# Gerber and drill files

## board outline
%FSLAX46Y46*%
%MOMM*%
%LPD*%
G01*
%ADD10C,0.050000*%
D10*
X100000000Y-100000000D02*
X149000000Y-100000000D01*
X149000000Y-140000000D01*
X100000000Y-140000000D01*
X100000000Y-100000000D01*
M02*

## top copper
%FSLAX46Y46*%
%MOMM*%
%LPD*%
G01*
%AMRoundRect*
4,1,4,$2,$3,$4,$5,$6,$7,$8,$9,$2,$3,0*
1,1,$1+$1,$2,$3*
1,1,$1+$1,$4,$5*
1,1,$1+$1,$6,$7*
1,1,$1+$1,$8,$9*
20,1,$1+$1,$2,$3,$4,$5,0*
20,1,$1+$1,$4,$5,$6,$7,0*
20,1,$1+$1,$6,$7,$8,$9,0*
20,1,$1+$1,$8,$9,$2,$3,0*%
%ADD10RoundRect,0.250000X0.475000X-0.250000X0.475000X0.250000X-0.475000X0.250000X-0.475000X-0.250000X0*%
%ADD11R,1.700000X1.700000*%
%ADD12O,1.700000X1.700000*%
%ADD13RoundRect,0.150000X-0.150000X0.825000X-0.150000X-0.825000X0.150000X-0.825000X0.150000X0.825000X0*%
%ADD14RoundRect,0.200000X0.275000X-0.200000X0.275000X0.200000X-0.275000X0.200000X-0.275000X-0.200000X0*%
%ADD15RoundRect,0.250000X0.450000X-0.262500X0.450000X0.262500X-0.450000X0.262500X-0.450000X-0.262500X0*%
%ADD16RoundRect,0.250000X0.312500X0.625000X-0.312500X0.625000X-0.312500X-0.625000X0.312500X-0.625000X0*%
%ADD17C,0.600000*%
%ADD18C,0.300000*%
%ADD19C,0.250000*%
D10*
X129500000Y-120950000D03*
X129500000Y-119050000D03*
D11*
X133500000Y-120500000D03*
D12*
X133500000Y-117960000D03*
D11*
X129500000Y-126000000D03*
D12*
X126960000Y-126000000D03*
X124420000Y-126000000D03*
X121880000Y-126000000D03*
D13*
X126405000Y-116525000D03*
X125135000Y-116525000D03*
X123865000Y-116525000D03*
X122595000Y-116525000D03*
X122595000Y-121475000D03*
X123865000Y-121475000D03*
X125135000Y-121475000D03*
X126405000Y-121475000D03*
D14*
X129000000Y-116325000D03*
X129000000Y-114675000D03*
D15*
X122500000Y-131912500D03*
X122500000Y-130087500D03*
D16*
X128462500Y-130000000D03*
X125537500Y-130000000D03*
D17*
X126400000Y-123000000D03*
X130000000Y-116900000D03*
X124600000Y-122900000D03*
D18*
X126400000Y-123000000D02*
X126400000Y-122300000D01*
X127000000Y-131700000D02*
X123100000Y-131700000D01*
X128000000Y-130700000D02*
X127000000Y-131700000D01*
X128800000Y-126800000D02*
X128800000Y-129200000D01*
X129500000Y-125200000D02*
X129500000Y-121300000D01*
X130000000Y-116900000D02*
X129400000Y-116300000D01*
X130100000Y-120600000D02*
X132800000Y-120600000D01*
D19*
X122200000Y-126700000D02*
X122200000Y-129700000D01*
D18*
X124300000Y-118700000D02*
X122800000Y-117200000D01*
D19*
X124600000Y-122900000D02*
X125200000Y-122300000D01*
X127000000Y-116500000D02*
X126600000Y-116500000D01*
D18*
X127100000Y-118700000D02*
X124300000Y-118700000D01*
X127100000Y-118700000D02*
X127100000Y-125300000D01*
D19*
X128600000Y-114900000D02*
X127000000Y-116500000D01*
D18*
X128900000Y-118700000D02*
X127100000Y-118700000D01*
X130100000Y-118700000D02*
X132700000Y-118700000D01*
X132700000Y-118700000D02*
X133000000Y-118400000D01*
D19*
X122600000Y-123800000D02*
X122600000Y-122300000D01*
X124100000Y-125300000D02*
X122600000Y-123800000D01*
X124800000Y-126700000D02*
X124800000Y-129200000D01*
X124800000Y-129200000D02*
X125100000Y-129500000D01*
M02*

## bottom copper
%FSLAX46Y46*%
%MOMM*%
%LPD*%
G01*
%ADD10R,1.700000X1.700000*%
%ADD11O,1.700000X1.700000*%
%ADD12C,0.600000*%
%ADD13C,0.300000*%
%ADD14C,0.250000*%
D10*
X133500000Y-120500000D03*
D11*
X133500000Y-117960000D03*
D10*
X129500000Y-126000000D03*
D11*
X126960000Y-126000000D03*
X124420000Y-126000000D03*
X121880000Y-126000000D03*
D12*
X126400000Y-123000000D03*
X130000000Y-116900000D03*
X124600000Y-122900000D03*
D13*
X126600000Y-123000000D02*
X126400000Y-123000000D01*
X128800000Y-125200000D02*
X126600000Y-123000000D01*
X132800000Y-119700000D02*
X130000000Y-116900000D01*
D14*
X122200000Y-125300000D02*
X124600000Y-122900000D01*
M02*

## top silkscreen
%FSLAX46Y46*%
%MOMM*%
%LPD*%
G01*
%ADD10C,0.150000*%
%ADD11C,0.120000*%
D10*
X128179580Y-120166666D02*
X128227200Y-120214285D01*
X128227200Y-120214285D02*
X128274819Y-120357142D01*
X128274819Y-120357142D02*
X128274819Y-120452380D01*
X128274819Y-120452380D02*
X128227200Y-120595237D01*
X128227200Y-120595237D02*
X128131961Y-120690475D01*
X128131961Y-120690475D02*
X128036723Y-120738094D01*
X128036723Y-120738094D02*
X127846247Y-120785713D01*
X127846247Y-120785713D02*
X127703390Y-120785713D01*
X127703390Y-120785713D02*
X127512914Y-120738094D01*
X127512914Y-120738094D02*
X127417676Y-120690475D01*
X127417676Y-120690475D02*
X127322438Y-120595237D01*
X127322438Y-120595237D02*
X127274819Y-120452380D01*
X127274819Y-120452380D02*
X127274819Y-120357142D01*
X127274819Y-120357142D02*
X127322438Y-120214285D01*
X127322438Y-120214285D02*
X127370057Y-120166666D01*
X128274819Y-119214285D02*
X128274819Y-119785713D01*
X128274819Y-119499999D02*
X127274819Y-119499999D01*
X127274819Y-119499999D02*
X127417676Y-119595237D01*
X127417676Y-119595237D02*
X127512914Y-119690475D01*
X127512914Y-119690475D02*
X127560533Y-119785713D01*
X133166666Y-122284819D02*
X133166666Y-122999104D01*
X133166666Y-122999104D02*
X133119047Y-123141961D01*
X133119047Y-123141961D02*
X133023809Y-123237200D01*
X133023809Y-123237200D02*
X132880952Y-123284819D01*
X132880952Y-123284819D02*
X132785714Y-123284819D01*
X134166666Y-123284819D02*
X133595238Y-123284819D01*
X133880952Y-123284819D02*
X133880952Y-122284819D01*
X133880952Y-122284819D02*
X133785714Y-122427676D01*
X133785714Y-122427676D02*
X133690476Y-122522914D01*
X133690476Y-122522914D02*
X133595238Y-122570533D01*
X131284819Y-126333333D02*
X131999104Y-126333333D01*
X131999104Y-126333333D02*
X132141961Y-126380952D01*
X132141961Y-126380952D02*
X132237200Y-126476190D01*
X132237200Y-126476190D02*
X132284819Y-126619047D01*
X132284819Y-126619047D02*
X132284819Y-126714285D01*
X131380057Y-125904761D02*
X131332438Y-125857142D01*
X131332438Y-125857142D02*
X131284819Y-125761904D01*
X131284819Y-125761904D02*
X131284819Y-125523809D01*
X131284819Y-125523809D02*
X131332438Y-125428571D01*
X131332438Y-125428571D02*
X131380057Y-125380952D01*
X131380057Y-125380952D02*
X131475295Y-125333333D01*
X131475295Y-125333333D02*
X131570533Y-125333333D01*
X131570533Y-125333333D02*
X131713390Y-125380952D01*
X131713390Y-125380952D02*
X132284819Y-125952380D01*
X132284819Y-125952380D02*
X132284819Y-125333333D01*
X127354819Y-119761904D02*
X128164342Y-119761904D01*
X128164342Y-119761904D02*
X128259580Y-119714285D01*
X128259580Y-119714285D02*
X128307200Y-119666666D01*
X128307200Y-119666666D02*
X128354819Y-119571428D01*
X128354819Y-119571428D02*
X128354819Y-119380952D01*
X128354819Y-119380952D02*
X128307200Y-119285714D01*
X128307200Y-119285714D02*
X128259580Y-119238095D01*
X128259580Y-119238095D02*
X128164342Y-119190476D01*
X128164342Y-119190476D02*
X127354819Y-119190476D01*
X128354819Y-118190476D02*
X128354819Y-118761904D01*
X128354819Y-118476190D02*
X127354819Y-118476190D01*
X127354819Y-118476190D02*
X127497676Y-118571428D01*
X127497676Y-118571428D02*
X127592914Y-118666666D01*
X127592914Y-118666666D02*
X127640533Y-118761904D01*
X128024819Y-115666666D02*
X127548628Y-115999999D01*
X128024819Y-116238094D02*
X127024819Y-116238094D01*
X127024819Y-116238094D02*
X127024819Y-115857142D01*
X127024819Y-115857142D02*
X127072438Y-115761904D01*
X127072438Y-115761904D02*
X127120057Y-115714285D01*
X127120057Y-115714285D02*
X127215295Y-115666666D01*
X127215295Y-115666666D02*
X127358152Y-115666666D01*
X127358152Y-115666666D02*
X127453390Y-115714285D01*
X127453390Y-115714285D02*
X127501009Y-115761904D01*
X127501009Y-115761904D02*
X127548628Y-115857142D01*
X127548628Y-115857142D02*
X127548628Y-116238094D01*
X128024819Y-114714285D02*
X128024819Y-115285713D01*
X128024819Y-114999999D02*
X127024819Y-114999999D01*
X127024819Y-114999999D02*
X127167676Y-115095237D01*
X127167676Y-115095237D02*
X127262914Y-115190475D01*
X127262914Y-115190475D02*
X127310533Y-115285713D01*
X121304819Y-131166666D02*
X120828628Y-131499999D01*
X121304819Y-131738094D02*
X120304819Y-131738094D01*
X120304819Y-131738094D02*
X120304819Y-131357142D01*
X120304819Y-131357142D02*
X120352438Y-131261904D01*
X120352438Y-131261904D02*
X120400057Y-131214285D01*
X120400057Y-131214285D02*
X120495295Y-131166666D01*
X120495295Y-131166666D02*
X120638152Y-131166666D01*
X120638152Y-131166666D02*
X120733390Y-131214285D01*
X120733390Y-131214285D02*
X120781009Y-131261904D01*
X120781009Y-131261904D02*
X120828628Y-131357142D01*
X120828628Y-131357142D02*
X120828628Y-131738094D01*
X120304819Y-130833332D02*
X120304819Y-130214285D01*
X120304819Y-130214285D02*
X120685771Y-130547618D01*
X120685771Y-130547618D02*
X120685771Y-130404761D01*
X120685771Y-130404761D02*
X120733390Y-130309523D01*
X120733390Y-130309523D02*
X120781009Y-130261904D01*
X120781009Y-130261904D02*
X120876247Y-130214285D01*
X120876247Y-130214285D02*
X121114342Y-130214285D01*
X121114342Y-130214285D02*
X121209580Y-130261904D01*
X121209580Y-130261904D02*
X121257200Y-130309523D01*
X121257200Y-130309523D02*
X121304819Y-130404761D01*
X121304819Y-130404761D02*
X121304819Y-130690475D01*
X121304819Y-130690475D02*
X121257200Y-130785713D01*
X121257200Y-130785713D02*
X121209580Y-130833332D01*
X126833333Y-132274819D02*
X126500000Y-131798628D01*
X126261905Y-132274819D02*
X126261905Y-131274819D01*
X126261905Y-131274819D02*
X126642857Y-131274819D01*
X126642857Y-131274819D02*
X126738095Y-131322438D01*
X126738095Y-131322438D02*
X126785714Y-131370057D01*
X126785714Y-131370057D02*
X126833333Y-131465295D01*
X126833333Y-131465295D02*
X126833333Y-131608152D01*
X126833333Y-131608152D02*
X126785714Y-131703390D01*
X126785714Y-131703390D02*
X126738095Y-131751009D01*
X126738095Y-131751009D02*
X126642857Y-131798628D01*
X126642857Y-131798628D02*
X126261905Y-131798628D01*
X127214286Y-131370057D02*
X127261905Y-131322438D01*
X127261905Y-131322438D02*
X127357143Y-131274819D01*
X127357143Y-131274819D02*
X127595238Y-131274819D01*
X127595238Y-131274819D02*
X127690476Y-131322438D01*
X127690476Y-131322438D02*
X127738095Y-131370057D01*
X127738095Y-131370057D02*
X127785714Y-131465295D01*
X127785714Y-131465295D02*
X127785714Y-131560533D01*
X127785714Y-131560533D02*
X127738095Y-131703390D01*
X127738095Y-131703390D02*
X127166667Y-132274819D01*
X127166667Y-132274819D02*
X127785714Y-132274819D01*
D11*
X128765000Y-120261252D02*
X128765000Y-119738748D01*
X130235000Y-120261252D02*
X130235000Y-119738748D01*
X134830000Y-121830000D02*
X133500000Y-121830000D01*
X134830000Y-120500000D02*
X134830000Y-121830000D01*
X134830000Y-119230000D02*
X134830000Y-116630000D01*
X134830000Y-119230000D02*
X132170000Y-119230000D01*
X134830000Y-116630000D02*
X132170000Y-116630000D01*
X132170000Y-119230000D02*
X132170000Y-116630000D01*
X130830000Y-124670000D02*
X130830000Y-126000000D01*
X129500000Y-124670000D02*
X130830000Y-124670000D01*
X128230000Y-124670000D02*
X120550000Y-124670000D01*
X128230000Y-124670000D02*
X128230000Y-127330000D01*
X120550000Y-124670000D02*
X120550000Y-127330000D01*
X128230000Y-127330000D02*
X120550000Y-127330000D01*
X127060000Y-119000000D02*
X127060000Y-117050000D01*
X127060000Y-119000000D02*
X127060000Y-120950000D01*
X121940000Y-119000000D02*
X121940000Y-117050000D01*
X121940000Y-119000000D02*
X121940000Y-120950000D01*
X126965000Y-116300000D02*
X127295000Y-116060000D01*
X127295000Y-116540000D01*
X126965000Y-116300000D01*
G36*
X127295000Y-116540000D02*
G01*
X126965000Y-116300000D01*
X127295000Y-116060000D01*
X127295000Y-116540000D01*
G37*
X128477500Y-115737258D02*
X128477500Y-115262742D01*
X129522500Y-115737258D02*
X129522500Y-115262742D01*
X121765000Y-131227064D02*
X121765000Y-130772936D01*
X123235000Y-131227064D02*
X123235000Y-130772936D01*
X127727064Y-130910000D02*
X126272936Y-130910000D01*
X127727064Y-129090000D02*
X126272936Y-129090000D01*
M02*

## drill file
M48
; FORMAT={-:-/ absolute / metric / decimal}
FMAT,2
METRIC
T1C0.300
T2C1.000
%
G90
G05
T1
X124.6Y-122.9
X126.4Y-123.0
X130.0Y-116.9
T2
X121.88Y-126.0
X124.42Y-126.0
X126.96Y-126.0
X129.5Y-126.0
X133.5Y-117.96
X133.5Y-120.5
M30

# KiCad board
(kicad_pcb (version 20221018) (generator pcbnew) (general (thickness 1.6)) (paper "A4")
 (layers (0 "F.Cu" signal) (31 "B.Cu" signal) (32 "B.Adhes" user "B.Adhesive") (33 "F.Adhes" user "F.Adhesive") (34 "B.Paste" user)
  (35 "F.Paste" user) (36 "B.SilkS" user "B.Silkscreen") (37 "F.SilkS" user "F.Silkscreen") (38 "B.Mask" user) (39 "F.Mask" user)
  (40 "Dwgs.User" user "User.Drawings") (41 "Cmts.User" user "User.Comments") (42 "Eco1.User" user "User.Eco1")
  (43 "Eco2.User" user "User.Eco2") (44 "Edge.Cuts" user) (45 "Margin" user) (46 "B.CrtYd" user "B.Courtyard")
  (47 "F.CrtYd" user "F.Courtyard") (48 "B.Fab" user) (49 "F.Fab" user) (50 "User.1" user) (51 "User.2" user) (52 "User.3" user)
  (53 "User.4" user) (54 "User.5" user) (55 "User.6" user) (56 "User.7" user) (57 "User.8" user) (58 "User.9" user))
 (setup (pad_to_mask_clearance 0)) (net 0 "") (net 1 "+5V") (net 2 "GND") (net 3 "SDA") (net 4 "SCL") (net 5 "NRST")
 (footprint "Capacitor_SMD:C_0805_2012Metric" (layer "F.Cu") (at 129.5 120 90)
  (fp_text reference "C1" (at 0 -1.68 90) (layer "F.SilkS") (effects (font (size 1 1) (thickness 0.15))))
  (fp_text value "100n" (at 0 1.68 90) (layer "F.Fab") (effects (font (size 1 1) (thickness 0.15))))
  (fp_line (start -0.261252 -0.735) (end 0.261252 -0.735) (stroke (width 0.12) (type solid)) (layer "F.SilkS"))
  (fp_line (start -0.261252 0.735) (end 0.261252 0.735) (stroke (width 0.12) (type solid)) (layer "F.SilkS"))
  (pad "1" smd roundrect (at -0.95 0 90) (size 1 1.45) (layers "F.Cu" "F.Paste" "F.Mask") (roundrect_rratio 0.25) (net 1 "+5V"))
  (pad "2" smd roundrect (at 0.95 0 90) (size 1 1.45) (layers "F.Cu" "F.Paste" "F.Mask") (roundrect_rratio 0.25) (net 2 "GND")))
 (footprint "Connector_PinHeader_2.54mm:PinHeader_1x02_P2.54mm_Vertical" (layer "F.Cu") (at 133.5 120.5 180)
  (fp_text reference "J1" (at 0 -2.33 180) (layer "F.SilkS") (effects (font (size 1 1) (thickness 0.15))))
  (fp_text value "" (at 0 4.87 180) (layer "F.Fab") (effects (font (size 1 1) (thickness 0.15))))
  (fp_line (start -1.33 -1.33) (end 0 -1.33) (stroke (width 0.12) (type solid)) (layer "F.SilkS"))
  (fp_line (start -1.33 0) (end -1.33 -1.33) (stroke (width 0.12) (type solid)) (layer "F.SilkS"))
  (fp_line (start -1.33 1.27) (end -1.33 3.87) (stroke (width 0.12) (type solid)) (layer "F.SilkS"))
  (fp_line (start -1.33 1.27) (end 1.33 1.27) (stroke (width 0.12) (type solid)) (layer "F.SilkS"))
  (fp_line (start -1.33 3.87) (end 1.33 3.87) (stroke (width 0.12) (type solid)) (layer "F.SilkS"))
  (fp_line (start 1.33 1.27) (end 1.33 3.87) (stroke (width 0.12) (type solid)) (layer "F.SilkS"))
  (pad "1" thru_hole rect (at 0 0 180) (size 1.7 1.7) (drill 1) (layers "*.Cu" "*.Mask") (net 1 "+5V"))
  (pad "2" thru_hole oval (at 0 2.54 180) (size 1.7 1.7) (drill 1) (layers "*.Cu" "*.Mask") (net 2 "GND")))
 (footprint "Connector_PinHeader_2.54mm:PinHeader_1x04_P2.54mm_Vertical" (layer "F.Cu") (at 129.5 126 -90)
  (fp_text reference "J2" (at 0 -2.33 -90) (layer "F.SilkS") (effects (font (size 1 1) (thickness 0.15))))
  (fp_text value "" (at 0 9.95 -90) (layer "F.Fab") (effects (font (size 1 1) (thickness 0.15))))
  (fp_line (start -1.33 -1.33) (end 0 -1.33) (stroke (width 0.12) (type solid)) (layer "F.SilkS"))
  (fp_line (start -1.33 0) (end -1.33 -1.33) (stroke (width 0.12) (type solid)) (layer "F.SilkS"))
  (fp_line (start -1.33 1.27) (end -1.33 8.95) (stroke (width 0.12) (type solid)) (layer "F.SilkS"))
  (fp_line (start -1.33 1.27) (end 1.33 1.27) (stroke (width 0.12) (type solid)) (layer "F.SilkS"))
  (fp_line (start -1.33 8.95) (end 1.33 8.95) (stroke (width 0.12) (type solid)) (layer "F.SilkS"))
  (fp_line (start 1.33 1.27) (end 1.33 8.95) (stroke (width 0.12) (type solid)) (layer "F.SilkS"))
  (pad "1" thru_hole rect (at 0 0 270) (size 1.7 1.7) (drill 1) (layers "*.Cu" "*.Mask") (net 1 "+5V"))
  (pad "2" thru_hole oval (at 0 2.54 270) (size 1.7 1.7) (drill 1) (layers "*.Cu" "*.Mask") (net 2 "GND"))
  (pad "3" thru_hole oval (at 0 5.08 270) (size 1.7 1.7) (drill 1) (layers "*.Cu" "*.Mask") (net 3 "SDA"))
  (pad "4" thru_hole oval (at 0 7.62 270) (size 1.7 1.7) (drill 1) (layers "*.Cu" "*.Mask") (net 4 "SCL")))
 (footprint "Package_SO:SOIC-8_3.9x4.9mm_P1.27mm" (layer "F.Cu") (at 124.5 119 -90)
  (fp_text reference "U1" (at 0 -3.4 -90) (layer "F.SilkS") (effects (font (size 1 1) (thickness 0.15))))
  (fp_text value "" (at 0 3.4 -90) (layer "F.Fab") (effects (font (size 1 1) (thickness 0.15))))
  (fp_line (start 0 -2.56) (end -1.95 -2.56) (stroke (width 0.12) (type solid)) (layer "F.SilkS"))
  (fp_line (start 0 -2.56) (end 1.95 -2.56) (stroke (width 0.12) (type solid)) (layer "F.SilkS"))
  (fp_line (start 0 2.56) (end -1.95 2.56) (stroke (width 0.12) (type solid)) (layer "F.SilkS"))
  (fp_line (start 0 2.56) (end 1.95 2.56) (stroke (width 0.12) (type solid)) (layer "F.SilkS"))
  (fp_poly
   (pts (xy -2.7 -2.465) (xy -2.94 -2.795) (xy -2.46 -2.795) (xy -2.7 -2.465)) (stroke (width 0.12) (type solid)) (fill solid)
   (layer "F.SilkS"))
  (pad "1" smd roundrect (at -2.475 -1.905 270) (size 1.95 0.6) (layers "F.Cu" "F.Paste" "F.Mask") (roundrect_rratio 0.25) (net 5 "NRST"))
  (pad "2" smd roundrect (at -2.475 -0.635 270) (size 1.95 0.6) (layers "F.Cu" "F.Paste" "F.Mask") (roundrect_rratio 0.25))
  (pad "3" smd roundrect (at -2.475 0.635 270) (size 1.95 0.6) (layers "F.Cu" "F.Paste" "F.Mask") (roundrect_rratio 0.25))
  (pad "4" smd roundrect (at -2.475 1.905 270) (size 1.95 0.6) (layers "F.Cu" "F.Paste" "F.Mask") (roundrect_rratio 0.25) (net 2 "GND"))
  (pad "5" smd roundrect (at 2.475 1.905 270) (size 1.95 0.6) (layers "F.Cu" "F.Paste" "F.Mask") (roundrect_rratio 0.25) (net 3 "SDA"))
  (pad "6" smd roundrect (at 2.475 0.635 270) (size 1.95 0.6) (layers "F.Cu" "F.Paste" "F.Mask") (roundrect_rratio 0.25))
  (pad "7" smd roundrect (at 2.475 -0.635 270) (size 1.95 0.6) (layers "F.Cu" "F.Paste" "F.Mask") (roundrect_rratio 0.25) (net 4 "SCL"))
  (pad "8" smd roundrect (at 2.475 -1.905 270) (size 1.95 0.6) (layers "F.Cu" "F.Paste" "F.Mask") (roundrect_rratio 0.25) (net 1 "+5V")))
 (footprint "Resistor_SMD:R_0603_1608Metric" (layer "F.Cu") (at 129 115.5 90)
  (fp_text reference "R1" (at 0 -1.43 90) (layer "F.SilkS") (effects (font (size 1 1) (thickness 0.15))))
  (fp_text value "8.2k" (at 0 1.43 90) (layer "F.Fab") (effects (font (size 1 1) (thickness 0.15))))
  (fp_line (start -0.237258 -0.5225) (end 0.237258 -0.5225) (stroke (width 0.12) (type solid)) (layer "F.SilkS"))
  (fp_line (start -0.237258 0.5225) (end 0.237258 0.5225) (stroke (width 0.12) (type solid)) (layer "F.SilkS"))
  (pad "1" smd roundrect (at -0.825 0 90) (size 0.8 0.95) (layers "F.Cu" "F.Paste" "F.Mask") (roundrect_rratio 0.25) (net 1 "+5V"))
  (pad "2" smd roundrect (at 0.825 0 90) (size 0.8 0.95) (layers "F.Cu" "F.Paste" "F.Mask") (roundrect_rratio 0.25) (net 5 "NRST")))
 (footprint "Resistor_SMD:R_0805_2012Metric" (layer "F.Cu") (at 122.5 131 90)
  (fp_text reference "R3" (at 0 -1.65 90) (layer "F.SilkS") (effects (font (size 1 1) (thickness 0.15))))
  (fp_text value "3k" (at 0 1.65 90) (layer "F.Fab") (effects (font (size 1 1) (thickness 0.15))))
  (fp_line (start -0.227064 -0.735) (end 0.227064 -0.735) (stroke (width 0.12) (type solid)) (layer "F.SilkS"))
  (fp_line (start -0.227064 0.735) (end 0.227064 0.735) (stroke (width 0.12) (type solid)) (layer "F.SilkS"))
  (pad "1" smd roundrect (at -0.9125 0 90) (size 1.025 1.4) (layers "F.Cu" "F.Paste" "F.Mask") (roundrect_rratio 0.243902) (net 1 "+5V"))
  (pad "2" smd roundrect (at 0.9125 0 90) (size 1.025 1.4) (layers "F.Cu" "F.Paste" "F.Mask") (roundrect_rratio 0.243902) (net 4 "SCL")))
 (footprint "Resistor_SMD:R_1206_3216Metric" (layer "F.Cu") (at 127 130 180)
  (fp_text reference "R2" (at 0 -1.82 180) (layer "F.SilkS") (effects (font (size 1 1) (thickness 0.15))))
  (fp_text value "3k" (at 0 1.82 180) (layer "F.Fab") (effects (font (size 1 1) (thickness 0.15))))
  (fp_line (start -0.727064 -0.91) (end 0.727064 -0.91) (stroke (width 0.12) (type solid)) (layer "F.SilkS"))
  (fp_line (start -0.727064 0.91) (end 0.727064 0.91) (stroke (width 0.12) (type solid)) (layer "F.SilkS"))
  (pad "1" smd roundrect (at -1.4625 0 180) (size 1.125 1.75) (layers "F.Cu" "F.Paste" "F.Mask") (roundrect_rratio 0.222222) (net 1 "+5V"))
  (pad "2" smd roundrect (at 1.4625 0 180) (size 1.125 1.75) (layers "F.Cu" "F.Paste" "F.Mask") (roundrect_rratio 0.222222) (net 3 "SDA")))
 (gr_rect (start 100 100) (end 149 140) (stroke (width 0.05) (type default)) (fill none) (layer "Edge.Cuts"))
 (segment (start 126.4 123) (end 126.4 122.3) (width 0.3) (layer "F.Cu") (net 1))
 (segment (start 127 131.7) (end 123.1 131.7) (width 0.3) (layer "F.Cu") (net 1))
 (segment (start 128 130.7) (end 127 131.7) (width 0.3) (layer "F.Cu") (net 1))
 (segment (start 128.8 126.8) (end 128.8 129.2) (width 0.3) (layer "F.Cu") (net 1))
 (segment (start 129.5 125.2) (end 129.5 121.3) (width 0.3) (layer "F.Cu") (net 1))
 (segment (start 130 116.9) (end 129.4 116.3) (width 0.3) (layer "F.Cu") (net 1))
 (segment (start 130.1 120.6) (end 132.8 120.6) (width 0.3) (layer "F.Cu") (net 1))
 (via (at 126.4 123) (size 0.6) (drill 0.3) (layers "F.Cu" "B.Cu") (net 1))
 (via (at 130 116.9) (size 0.6) (drill 0.3) (layers "F.Cu" "B.Cu") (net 1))
 (segment (start 122.2 126.7) (end 122.2 129.7) (width 0.25) (layer "F.Cu") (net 4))
 (segment (start 124.3 118.7) (end 122.8 117.2) (width 0.3) (layer "F.Cu") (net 2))
 (segment (start 124.6 122.9) (end 125.2 122.3) (width 0.25) (layer "F.Cu") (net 4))
 (segment (start 126.6 123) (end 126.4 123) (width 0.3) (layer "B.Cu") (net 1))
 (segment (start 127 116.5) (end 126.6 116.5) (width 0.25) (layer "F.Cu") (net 5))
 (segment (start 127.1 118.7) (end 124.3 118.7) (width 0.3) (layer "F.Cu") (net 2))
 (segment (start 127.1 118.7) (end 127.1 125.3) (width 0.3) (layer "F.Cu") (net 2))
 (segment (start 128.6 114.9) (end 127 116.5) (width 0.25) (layer "F.Cu") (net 5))
 (segment (start 128.8 125.2) (end 126.6 123) (width 0.3) (layer "B.Cu") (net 1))
 (segment (start 128.9 118.7) (end 127.1 118.7) (width 0.3) (layer "F.Cu") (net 2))
 (segment (start 130.1 118.7) (end 132.7 118.7) (width 0.3) (layer "F.Cu") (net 2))
 (segment (start 132.7 118.7) (end 133 118.4) (width 0.3) (layer "F.Cu") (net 2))
 (segment (start 132.8 119.7) (end 130 116.9) (width 0.3) (layer "B.Cu") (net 1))
 (via (at 124.6 122.9) (size 0.6) (drill 0.3) (layers "F.Cu" "B.Cu") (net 4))
 (segment (start 122.2 125.3) (end 124.6 122.9) (width 0.25) (layer "B.Cu") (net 4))
 (segment (start 122.6 123.8) (end 122.6 122.3) (width 0.25) (layer "F.Cu") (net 3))
 (segment (start 124.1 125.3) (end 122.6 123.8) (width 0.25) (layer "F.Cu") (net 3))
 (segment (start 124.8 126.7) (end 124.8 129.2) (width 0.25) (layer "F.Cu") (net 3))
 (segment (start 124.8 129.2) (end 125.1 129.5) (width 0.25) (layer "F.Cu") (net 3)))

